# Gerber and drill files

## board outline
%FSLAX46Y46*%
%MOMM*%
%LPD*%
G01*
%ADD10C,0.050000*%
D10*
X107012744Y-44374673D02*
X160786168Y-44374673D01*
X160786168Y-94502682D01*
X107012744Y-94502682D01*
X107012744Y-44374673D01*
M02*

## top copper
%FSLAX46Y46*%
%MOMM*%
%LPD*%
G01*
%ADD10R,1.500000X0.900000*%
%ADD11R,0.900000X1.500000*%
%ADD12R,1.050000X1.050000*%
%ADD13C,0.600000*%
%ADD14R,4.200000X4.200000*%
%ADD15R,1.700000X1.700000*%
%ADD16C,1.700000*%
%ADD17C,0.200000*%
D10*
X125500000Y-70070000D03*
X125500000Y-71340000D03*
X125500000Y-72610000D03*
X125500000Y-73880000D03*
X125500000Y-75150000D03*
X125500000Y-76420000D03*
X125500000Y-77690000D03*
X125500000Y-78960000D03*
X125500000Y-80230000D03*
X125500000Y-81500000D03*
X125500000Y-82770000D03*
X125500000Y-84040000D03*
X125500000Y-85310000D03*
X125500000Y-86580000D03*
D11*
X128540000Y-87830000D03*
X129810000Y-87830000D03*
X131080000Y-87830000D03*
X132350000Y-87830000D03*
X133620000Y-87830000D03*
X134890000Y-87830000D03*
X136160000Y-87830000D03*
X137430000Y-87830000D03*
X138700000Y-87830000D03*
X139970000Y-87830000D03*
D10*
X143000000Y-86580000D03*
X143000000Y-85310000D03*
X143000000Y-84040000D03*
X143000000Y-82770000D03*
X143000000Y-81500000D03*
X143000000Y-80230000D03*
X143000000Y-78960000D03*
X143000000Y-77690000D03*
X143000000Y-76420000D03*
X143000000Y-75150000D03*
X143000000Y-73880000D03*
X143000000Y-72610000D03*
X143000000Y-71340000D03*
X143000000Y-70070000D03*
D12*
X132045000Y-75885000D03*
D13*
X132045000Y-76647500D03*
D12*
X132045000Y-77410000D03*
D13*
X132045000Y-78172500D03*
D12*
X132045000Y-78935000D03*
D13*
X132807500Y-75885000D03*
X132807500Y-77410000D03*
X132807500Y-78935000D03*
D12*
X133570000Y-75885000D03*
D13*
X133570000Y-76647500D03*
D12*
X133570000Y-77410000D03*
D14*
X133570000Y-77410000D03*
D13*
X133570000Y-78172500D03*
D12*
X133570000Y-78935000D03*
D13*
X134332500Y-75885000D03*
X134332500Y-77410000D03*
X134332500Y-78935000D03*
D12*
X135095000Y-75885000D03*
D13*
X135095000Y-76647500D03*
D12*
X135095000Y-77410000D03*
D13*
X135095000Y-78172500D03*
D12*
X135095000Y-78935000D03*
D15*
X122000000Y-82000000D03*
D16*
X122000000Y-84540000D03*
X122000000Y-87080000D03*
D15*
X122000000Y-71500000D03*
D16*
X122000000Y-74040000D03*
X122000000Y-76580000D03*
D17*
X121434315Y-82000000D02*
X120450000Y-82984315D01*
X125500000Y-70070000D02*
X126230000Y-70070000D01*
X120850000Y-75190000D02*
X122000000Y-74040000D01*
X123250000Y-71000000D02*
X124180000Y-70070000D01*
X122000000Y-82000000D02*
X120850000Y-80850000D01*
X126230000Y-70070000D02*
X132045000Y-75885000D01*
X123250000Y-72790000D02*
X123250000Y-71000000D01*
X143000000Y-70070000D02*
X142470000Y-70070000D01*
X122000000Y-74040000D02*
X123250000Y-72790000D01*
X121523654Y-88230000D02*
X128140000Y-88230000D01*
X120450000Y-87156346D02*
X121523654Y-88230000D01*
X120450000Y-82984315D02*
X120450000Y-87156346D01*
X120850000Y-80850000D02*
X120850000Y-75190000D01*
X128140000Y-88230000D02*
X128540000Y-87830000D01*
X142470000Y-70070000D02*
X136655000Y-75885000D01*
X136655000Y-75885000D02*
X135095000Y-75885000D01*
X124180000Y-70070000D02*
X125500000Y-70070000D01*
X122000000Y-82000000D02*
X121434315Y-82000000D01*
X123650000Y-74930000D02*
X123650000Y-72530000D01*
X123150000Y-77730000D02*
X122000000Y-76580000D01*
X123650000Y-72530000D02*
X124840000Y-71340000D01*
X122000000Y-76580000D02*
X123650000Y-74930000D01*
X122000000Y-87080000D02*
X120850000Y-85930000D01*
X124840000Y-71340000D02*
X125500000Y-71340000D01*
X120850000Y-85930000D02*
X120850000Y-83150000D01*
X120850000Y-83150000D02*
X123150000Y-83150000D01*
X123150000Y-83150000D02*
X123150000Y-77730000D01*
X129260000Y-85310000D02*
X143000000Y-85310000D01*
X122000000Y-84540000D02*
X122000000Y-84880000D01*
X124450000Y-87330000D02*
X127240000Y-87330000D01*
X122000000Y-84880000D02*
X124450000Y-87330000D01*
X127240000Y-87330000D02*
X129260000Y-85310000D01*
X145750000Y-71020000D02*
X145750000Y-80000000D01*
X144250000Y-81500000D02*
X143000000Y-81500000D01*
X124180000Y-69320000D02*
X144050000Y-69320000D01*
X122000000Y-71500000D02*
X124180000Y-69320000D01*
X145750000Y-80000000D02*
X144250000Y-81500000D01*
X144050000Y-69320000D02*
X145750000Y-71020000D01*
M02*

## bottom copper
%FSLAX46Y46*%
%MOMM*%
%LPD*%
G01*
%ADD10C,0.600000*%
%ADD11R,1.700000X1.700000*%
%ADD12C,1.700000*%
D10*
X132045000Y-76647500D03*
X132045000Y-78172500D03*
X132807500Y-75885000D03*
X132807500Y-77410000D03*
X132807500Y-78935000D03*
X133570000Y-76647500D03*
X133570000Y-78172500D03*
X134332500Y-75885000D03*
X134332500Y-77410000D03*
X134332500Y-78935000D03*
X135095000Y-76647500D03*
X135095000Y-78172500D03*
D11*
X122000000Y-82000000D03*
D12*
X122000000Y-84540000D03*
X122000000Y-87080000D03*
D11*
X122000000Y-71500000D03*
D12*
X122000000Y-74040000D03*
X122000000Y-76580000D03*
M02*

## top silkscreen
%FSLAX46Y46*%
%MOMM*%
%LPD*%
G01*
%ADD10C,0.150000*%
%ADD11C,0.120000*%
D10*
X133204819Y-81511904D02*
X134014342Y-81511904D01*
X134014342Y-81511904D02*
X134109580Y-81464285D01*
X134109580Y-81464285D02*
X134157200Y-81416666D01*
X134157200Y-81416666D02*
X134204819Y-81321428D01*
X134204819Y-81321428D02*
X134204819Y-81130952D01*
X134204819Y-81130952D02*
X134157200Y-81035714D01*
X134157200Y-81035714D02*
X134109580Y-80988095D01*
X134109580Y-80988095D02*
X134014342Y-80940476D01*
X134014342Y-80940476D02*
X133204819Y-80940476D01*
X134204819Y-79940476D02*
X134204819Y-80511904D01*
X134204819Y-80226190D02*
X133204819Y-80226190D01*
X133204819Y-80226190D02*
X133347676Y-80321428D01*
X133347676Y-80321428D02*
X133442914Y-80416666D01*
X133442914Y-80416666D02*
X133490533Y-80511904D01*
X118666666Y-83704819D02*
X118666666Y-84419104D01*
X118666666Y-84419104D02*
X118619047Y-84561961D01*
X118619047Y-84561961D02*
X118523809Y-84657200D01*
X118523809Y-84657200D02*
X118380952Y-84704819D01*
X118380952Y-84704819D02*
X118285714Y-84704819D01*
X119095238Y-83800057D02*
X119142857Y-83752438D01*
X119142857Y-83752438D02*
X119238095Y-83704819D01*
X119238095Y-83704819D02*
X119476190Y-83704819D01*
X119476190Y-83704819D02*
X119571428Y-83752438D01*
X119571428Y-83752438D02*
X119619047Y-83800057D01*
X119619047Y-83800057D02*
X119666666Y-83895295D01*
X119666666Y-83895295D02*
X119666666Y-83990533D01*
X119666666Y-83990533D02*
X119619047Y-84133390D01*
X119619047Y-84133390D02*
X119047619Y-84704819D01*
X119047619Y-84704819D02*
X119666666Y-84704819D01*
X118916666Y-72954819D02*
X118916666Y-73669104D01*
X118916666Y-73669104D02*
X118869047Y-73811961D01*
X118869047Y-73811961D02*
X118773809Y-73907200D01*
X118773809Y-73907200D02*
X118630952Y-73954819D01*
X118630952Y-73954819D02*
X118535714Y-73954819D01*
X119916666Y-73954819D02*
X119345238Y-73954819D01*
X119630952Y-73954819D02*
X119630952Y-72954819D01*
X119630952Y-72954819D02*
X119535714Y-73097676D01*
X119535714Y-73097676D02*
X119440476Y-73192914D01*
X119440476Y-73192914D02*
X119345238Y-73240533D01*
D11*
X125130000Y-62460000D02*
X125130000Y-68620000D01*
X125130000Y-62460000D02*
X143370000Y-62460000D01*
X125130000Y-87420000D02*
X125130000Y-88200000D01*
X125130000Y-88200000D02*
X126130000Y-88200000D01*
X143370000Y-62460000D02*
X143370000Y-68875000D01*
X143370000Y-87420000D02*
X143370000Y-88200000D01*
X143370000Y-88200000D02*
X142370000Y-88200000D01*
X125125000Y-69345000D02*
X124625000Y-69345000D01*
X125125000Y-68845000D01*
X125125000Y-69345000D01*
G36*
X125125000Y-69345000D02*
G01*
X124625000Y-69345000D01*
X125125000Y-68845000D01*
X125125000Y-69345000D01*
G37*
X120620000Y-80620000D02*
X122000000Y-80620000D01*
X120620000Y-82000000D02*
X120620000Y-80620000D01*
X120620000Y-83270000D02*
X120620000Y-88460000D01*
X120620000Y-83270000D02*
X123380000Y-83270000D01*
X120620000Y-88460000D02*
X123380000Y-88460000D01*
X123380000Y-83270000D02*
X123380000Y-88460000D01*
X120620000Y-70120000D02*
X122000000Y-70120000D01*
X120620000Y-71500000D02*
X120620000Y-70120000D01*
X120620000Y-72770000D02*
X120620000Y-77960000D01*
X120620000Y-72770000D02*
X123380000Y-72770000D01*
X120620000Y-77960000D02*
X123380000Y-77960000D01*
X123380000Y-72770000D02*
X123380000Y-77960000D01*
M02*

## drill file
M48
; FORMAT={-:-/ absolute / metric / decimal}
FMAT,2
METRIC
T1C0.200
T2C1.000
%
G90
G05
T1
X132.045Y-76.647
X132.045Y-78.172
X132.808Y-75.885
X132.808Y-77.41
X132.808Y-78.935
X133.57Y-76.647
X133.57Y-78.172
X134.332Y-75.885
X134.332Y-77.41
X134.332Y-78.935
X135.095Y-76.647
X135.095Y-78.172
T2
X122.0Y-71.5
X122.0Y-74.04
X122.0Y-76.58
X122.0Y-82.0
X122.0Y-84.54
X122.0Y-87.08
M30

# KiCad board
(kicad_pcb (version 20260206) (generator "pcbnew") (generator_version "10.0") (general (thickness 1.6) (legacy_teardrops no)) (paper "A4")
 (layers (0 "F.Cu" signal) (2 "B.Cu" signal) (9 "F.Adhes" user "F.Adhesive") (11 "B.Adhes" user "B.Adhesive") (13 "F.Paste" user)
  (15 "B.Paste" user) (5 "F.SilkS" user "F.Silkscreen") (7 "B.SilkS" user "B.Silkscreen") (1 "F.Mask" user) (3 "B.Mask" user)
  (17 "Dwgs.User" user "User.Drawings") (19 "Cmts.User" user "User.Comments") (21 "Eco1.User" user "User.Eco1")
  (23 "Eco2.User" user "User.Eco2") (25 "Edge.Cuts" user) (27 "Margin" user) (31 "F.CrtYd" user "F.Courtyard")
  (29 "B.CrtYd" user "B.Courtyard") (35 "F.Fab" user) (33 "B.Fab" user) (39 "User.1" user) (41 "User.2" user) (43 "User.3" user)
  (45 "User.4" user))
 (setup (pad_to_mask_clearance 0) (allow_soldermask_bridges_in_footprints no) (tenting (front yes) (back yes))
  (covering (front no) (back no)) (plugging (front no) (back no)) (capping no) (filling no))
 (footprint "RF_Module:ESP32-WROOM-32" (layer "F.Cu") (at 134.25 78.32)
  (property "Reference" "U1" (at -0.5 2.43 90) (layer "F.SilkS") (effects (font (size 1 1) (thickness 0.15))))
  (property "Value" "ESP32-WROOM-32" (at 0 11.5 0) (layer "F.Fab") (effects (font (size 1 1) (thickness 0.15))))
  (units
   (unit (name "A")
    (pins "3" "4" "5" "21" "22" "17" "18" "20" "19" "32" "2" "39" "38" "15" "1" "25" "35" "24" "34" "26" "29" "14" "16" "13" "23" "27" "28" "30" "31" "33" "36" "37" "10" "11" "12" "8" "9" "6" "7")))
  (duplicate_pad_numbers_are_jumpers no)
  (fp_line (start -9.12 -15.86) (end -9.12 -9.7) (stroke (width 0.12) (type solid)) (layer "F.SilkS"))
  (fp_line (start -9.12 -15.86) (end 9.12 -15.86) (stroke (width 0.12) (type solid)) (layer "F.SilkS"))
  (fp_line (start -9.12 9.1) (end -9.12 9.88) (stroke (width 0.12) (type solid)) (layer "F.SilkS"))
  (fp_line (start -9.12 9.88) (end -8.12 9.88) (stroke (width 0.12) (type solid)) (layer "F.SilkS"))
  (fp_line (start 9.12 -15.86) (end 9.12 -9.445) (stroke (width 0.12) (type solid)) (layer "F.SilkS"))
  (fp_line (start 9.12 9.1) (end 9.12 9.88) (stroke (width 0.12) (type solid)) (layer "F.SilkS"))
  (fp_line (start 9.12 9.88) (end 8.12 9.88) (stroke (width 0.12) (type solid)) (layer "F.SilkS"))
  (fp_poly
   (pts (xy -9.125 -8.975) (xy -9.625 -8.975) (xy -9.125 -9.475) (xy -9.125 -8.975)) (stroke (width 0.12) (type solid)) (fill yes)
   (layer "F.SilkS"))
  (pad "1" smd rect (at -8.75 -8.25) (size 1.5 0.9) (layers "F.Cu" "F.Mask" "F.Paste") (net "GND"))
  (pad "2" smd rect (at -8.75 -6.98) (size 1.5 0.9) (layers "F.Cu" "F.Mask" "F.Paste") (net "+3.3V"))
  (pad "3" smd rect (at -8.75 -5.71) (size 1.5 0.9) (layers "F.Cu" "F.Mask" "F.Paste") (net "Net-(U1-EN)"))
  (pad "4" smd rect (at -8.75 -4.44) (size 1.5 0.9) (layers "F.Cu" "F.Mask" "F.Paste") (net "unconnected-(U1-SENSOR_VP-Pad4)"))
  (pad "5" smd rect (at -8.75 -3.17) (size 1.5 0.9) (layers "F.Cu" "F.Mask" "F.Paste") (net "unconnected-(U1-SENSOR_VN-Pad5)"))
  (pad "6" smd rect (at -8.75 -1.9) (size 1.5 0.9) (layers "F.Cu" "F.Mask" "F.Paste") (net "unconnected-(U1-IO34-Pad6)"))
  (pad "7" smd rect (at -8.75 -0.63) (size 1.5 0.9) (layers "F.Cu" "F.Mask" "F.Paste") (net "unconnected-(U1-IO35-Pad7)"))
  (pad "8" smd rect (at -8.75 0.64) (size 1.5 0.9) (layers "F.Cu" "F.Mask" "F.Paste") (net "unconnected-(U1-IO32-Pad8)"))
  (pad "9" smd rect (at -8.75 1.91) (size 1.5 0.9) (layers "F.Cu" "F.Mask" "F.Paste") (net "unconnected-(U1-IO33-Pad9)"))
  (pad "10" smd rect (at -8.75 3.18) (size 1.5 0.9) (layers "F.Cu" "F.Mask" "F.Paste") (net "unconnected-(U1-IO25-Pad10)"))
  (pad "11" smd rect (at -8.75 4.45) (size 1.5 0.9) (layers "F.Cu" "F.Mask" "F.Paste") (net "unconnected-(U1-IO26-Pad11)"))
  (pad "12" smd rect (at -8.75 5.72) (size 1.5 0.9) (layers "F.Cu" "F.Mask" "F.Paste") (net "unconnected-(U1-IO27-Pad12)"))
  (pad "13" smd rect (at -8.75 6.99) (size 1.5 0.9) (layers "F.Cu" "F.Mask" "F.Paste") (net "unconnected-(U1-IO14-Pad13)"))
  (pad "14" smd rect (at -8.75 8.26) (size 1.5 0.9) (layers "F.Cu" "F.Mask" "F.Paste") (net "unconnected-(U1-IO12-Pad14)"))
  (pad "15" smd rect (at -5.71 9.51 90) (size 1.5 0.9) (layers "F.Cu" "F.Mask" "F.Paste") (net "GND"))
  (pad "16" smd rect (at -4.44 9.51 90) (size 1.5 0.9) (layers "F.Cu" "F.Mask" "F.Paste") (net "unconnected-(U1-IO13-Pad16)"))
  (pad "17" smd rect (at -3.17 9.51 90) (size 1.5 0.9) (layers "F.Cu" "F.Mask" "F.Paste") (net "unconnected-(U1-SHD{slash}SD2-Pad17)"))
  (pad "18" smd rect (at -1.9 9.51 90) (size 1.5 0.9) (layers "F.Cu" "F.Mask" "F.Paste") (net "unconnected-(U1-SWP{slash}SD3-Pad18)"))
  (pad "19" smd rect (at -0.63 9.51 90) (size 1.5 0.9) (layers "F.Cu" "F.Mask" "F.Paste") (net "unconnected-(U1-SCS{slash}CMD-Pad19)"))
  (pad "20" smd rect (at 0.64 9.51 90) (size 1.5 0.9) (layers "F.Cu" "F.Mask" "F.Paste") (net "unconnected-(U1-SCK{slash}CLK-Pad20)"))
  (pad "21" smd rect (at 1.91 9.51 90) (size 1.5 0.9) (layers "F.Cu" "F.Mask" "F.Paste") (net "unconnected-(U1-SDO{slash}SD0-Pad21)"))
  (pad "22" smd rect (at 3.18 9.51 90) (size 1.5 0.9) (layers "F.Cu" "F.Mask" "F.Paste") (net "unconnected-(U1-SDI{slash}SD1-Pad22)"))
  (pad "23" smd rect (at 4.45 9.51 90) (size 1.5 0.9) (layers "F.Cu" "F.Mask" "F.Paste") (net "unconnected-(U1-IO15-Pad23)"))
  (pad "24" smd rect (at 5.72 9.51 90) (size 1.5 0.9) (layers "F.Cu" "F.Mask" "F.Paste") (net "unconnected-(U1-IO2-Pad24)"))
  (pad "25" smd rect (at 8.75 8.26) (size 1.5 0.9) (layers "F.Cu" "F.Mask" "F.Paste") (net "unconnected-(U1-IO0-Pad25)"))
  (pad "26" smd rect (at 8.75 6.99) (size 1.5 0.9) (layers "F.Cu" "F.Mask" "F.Paste") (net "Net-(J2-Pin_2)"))
  (pad "27" smd rect (at 8.75 5.72) (size 1.5 0.9) (layers "F.Cu" "F.Mask" "F.Paste") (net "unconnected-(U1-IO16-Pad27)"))
  (pad "28" smd rect (at 8.75 4.45) (size 1.5 0.9) (layers "F.Cu" "F.Mask" "F.Paste") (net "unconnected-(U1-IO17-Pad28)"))
  (pad "29" smd rect (at 8.75 3.18) (size 1.5 0.9) (layers "F.Cu" "F.Mask" "F.Paste") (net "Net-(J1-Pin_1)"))
  (pad "30" smd rect (at 8.75 1.91) (size 1.5 0.9) (layers "F.Cu" "F.Mask" "F.Paste") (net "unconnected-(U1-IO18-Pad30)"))
  (pad "31" smd rect (at 8.75 0.64) (size 1.5 0.9) (layers "F.Cu" "F.Mask" "F.Paste") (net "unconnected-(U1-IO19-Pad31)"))
  (pad "32" smd rect (at 8.75 -0.63) (size 1.5 0.9) (layers "F.Cu" "F.Mask" "F.Paste") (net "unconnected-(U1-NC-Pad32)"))
  (pad "33" smd rect (at 8.75 -1.9) (size 1.5 0.9) (layers "F.Cu" "F.Mask" "F.Paste") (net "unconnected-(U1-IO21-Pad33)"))
  (pad "34" smd rect (at 8.75 -3.17) (size 1.5 0.9) (layers "F.Cu" "F.Mask" "F.Paste") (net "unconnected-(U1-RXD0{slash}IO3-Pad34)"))
  (pad "35" smd rect (at 8.75 -4.44) (size 1.5 0.9) (layers "F.Cu" "F.Mask" "F.Paste") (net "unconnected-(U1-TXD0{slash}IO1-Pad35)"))
  (pad "36" smd rect (at 8.75 -5.71) (size 1.5 0.9) (layers "F.Cu" "F.Mask" "F.Paste") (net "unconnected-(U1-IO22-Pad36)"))
  (pad "37" smd rect (at 8.75 -6.98) (size 1.5 0.9) (layers "F.Cu" "F.Mask" "F.Paste") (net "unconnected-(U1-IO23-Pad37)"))
  (pad "38" smd rect (at 8.75 -8.25) (size 1.5 0.9) (layers "F.Cu" "F.Mask" "F.Paste") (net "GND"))
  (pad "39" smd rect (at -2.205 -2.435) (size 1.05 1.05) (layers "F.Cu" "F.Paste") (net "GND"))
  (pad "39" thru_hole circle (at -2.205 -1.6725) (size 0.6 0.6) (drill 0.2) (layers "*.Cu" "F.Mask") (remove_unused_layers no) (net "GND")
   (zone_connect 2))
  (pad "39" smd rect (at -2.205 -0.91) (size 1.05 1.05) (layers "F.Cu" "F.Paste") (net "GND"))
  (pad "39" thru_hole circle (at -2.205 -0.1475) (size 0.6 0.6) (drill 0.2) (layers "*.Cu" "F.Mask") (remove_unused_layers no) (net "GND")
   (zone_connect 2))
  (pad "39" smd rect (at -2.205 0.615) (size 1.05 1.05) (layers "F.Cu" "F.Paste") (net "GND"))
  (pad "39" thru_hole circle (at -1.4425 -2.435) (size 0.6 0.6) (drill 0.2) (layers "*.Cu" "F.Mask") (remove_unused_layers no) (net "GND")
   (zone_connect 2))
  (pad "39" thru_hole circle (at -1.4425 -0.91) (size 0.6 0.6) (drill 0.2) (layers "*.Cu" "F.Mask") (remove_unused_layers no) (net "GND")
   (zone_connect 2))
  (pad "39" thru_hole circle (at -1.4425 0.615) (size 0.6 0.6) (drill 0.2) (layers "*.Cu" "F.Mask") (remove_unused_layers no) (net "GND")
   (zone_connect 2))
  (pad "39" smd rect (at -0.68 -2.435) (size 1.05 1.05) (layers "F.Cu" "F.Paste") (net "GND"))
  (pad "39" thru_hole circle (at -0.68 -1.6725) (size 0.6 0.6) (drill 0.2) (layers "*.Cu" "F.Mask") (remove_unused_layers no) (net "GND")
   (zone_connect 2))
  (pad "39" smd rect (at -0.68 -0.91) (size 1.05 1.05) (layers "F.Cu" "F.Paste") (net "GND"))
  (pad "39" smd rect (at -0.68 -0.91) (size 4.2 4.2) (layers "F.Cu" "F.Mask") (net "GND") (zone_connect 2))
  (pad "39" thru_hole circle (at -0.68 -0.1475) (size 0.6 0.6) (drill 0.2) (layers "*.Cu" "F.Mask") (remove_unused_layers no) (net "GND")
   (zone_connect 2))
  (pad "39" smd rect (at -0.68 0.615) (size 1.05 1.05) (layers "F.Cu" "F.Paste") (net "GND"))
  (pad "39" thru_hole circle (at 0.0825 -2.435) (size 0.6 0.6) (drill 0.2) (layers "*.Cu" "F.Mask") (remove_unused_layers no) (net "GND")
   (zone_connect 2))
  (pad "39" thru_hole circle (at 0.0825 -0.91) (size 0.6 0.6) (drill 0.2) (layers "*.Cu" "F.Mask") (remove_unused_layers no) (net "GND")
   (zone_connect 2))
  (pad "39" thru_hole circle (at 0.0825 0.615) (size 0.6 0.6) (drill 0.2) (layers "*.Cu" "F.Mask") (remove_unused_layers no) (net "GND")
   (zone_connect 2))
  (pad "39" smd rect (at 0.845 -2.435) (size 1.05 1.05) (layers "F.Cu" "F.Paste") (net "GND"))
  (pad "39" thru_hole circle (at 0.845 -1.6725) (size 0.6 0.6) (drill 0.2) (layers "*.Cu" "F.Mask") (remove_unused_layers no) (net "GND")
   (zone_connect 2))
  (pad "39" smd rect (at 0.845 -0.91) (size 1.05 1.05) (layers "F.Cu" "F.Paste") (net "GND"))
  (pad "39" thru_hole circle (at 0.845 -0.1475) (size 0.6 0.6) (drill 0.2) (layers "*.Cu" "F.Mask") (remove_unused_layers no) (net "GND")
   (zone_connect 2))
  (pad "39" smd rect (at 0.845 0.615) (size 1.05 1.05) (layers "F.Cu" "F.Paste") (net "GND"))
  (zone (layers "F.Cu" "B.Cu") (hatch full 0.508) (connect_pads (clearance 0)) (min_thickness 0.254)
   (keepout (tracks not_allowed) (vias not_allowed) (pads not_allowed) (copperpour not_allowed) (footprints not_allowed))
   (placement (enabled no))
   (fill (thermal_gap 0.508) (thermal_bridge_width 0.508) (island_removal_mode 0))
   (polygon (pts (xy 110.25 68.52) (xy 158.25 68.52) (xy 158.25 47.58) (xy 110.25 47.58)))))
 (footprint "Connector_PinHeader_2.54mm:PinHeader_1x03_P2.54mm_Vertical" (layer "F.Cu") (at 122 82)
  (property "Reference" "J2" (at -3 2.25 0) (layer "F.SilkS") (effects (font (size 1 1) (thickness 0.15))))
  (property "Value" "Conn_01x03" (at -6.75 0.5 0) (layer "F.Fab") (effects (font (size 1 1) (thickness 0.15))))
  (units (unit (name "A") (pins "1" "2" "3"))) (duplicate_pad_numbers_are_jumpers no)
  (fp_line (start -1.38 -1.38) (end 0 -1.38) (stroke (width 0.12) (type solid)) (layer "F.SilkS"))
  (fp_line (start -1.38 0) (end -1.38 -1.38) (stroke (width 0.12) (type solid)) (layer "F.SilkS"))
  (fp_line (start -1.38 1.27) (end -1.38 6.46) (stroke (width 0.12) (type solid)) (layer "F.SilkS"))
  (fp_line (start -1.38 1.27) (end 1.38 1.27) (stroke (width 0.12) (type solid)) (layer "F.SilkS"))
  (fp_line (start -1.38 6.46) (end 1.38 6.46) (stroke (width 0.12) (type solid)) (layer "F.SilkS"))
  (fp_line (start 1.38 1.27) (end 1.38 6.46) (stroke (width 0.12) (type solid)) (layer "F.SilkS"))
  (pad "1" thru_hole rect (at 0 0) (size 1.7 1.7) (drill 1) (layers "*.Cu" "*.Mask") (remove_unused_layers no) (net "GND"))
  (pad "2" thru_hole circle (at 0 2.54) (size 1.7 1.7) (drill 1) (layers "*.Cu" "*.Mask") (remove_unused_layers no) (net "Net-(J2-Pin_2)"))
  (pad "3" thru_hole circle (at 0 5.08) (size 1.7 1.7) (drill 1) (layers "*.Cu" "*.Mask") (remove_unused_layers no) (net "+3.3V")))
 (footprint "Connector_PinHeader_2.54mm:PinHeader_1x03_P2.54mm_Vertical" (layer "F.Cu") (at 122 71.5)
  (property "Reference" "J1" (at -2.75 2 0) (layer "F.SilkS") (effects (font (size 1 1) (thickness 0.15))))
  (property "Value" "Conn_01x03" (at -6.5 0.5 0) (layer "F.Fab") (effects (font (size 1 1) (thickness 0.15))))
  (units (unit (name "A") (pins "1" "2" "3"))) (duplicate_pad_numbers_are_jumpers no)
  (fp_line (start -1.38 -1.38) (end 0 -1.38) (stroke (width 0.12) (type solid)) (layer "F.SilkS"))
  (fp_line (start -1.38 0) (end -1.38 -1.38) (stroke (width 0.12) (type solid)) (layer "F.SilkS"))
  (fp_line (start -1.38 1.27) (end -1.38 6.46) (stroke (width 0.12) (type solid)) (layer "F.SilkS"))
  (fp_line (start -1.38 1.27) (end 1.38 1.27) (stroke (width 0.12) (type solid)) (layer "F.SilkS"))
  (fp_line (start -1.38 6.46) (end 1.38 6.46) (stroke (width 0.12) (type solid)) (layer "F.SilkS"))
  (fp_line (start 1.38 1.27) (end 1.38 6.46) (stroke (width 0.12) (type solid)) (layer "F.SilkS"))
  (pad "1" thru_hole rect (at 0 0) (size 1.7 1.7) (drill 1) (layers "*.Cu" "*.Mask") (remove_unused_layers no) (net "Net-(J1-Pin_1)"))
  (pad "2" thru_hole circle (at 0 2.54) (size 1.7 1.7) (drill 1) (layers "*.Cu" "*.Mask") (remove_unused_layers no) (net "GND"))
  (pad "3" thru_hole circle (at 0 5.08) (size 1.7 1.7) (drill 1) (layers "*.Cu" "*.Mask") (remove_unused_layers no) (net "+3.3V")))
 (gr_rect (start 107.012744 44.374673) (end 160.786168 94.502682) (stroke (width 0.05) (type default)) (fill no) (layer "Edge.Cuts"))
 (segment (start 121.434315 82) (end 120.45 82.984315) (width 0.2) (layer "F.Cu") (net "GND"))
 (segment (start 125.5 70.07) (end 126.23 70.07) (width 0.2) (layer "F.Cu") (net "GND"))
 (segment (start 120.85 75.19) (end 122 74.04) (width 0.2) (layer "F.Cu") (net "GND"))
 (segment (start 123.25 71) (end 124.18 70.07) (width 0.2) (layer "F.Cu") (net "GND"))
 (segment (start 122 82) (end 120.85 80.85) (width 0.2) (layer "F.Cu") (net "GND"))
 (segment (start 126.23 70.07) (end 132.045 75.885) (width 0.2) (layer "F.Cu") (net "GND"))
 (segment (start 123.25 72.79) (end 123.25 71) (width 0.2) (layer "F.Cu") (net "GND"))
 (segment (start 143 70.07) (end 142.47 70.07) (width 0.2) (layer "F.Cu") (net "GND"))
 (segment (start 122 74.04) (end 123.25 72.79) (width 0.2) (layer "F.Cu") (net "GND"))
 (segment (start 121.523654 88.23) (end 128.14 88.23) (width 0.2) (layer "F.Cu") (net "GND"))
 (segment (start 120.45 87.156346) (end 121.523654 88.23) (width 0.2) (layer "F.Cu") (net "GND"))
 (segment (start 120.45 82.984315) (end 120.45 87.156346) (width 0.2) (layer "F.Cu") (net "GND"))
 (segment (start 120.85 80.85) (end 120.85 75.19) (width 0.2) (layer "F.Cu") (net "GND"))
 (segment (start 128.14 88.23) (end 128.54 87.83) (width 0.2) (layer "F.Cu") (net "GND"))
 (segment (start 142.47 70.07) (end 136.655 75.885) (width 0.2) (layer "F.Cu") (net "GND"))
 (segment (start 136.655 75.885) (end 135.095 75.885) (width 0.2) (layer "F.Cu") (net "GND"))
 (segment (start 124.18 70.07) (end 125.5 70.07) (width 0.2) (layer "F.Cu") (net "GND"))
 (segment (start 122 82) (end 121.434315 82) (width 0.2) (layer "F.Cu") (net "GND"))
 (segment (start 123.65 74.93) (end 123.65 72.53) (width 0.2) (layer "F.Cu") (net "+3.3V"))
 (segment (start 123.15 77.73) (end 122 76.58) (width 0.2) (layer "F.Cu") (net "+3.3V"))
 (segment (start 123.65 72.53) (end 124.84 71.34) (width 0.2) (layer "F.Cu") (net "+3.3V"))
 (segment (start 122 76.58) (end 123.65 74.93) (width 0.2) (layer "F.Cu") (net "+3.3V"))
 (segment (start 122 87.08) (end 120.85 85.93) (width 0.2) (layer "F.Cu") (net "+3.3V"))
 (segment (start 124.84 71.34) (end 125.5 71.34) (width 0.2) (layer "F.Cu") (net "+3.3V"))
 (segment (start 120.85 85.93) (end 120.85 83.15) (width 0.2) (layer "F.Cu") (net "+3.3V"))
 (segment (start 120.85 83.15) (end 123.15 83.15) (width 0.2) (layer "F.Cu") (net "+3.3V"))
 (segment (start 123.15 83.15) (end 123.15 77.73) (width 0.2) (layer "F.Cu") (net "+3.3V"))
 (segment (start 129.26 85.31) (end 143 85.31) (width 0.2) (layer "F.Cu") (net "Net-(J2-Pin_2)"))
 (segment (start 122 84.54) (end 122 84.88) (width 0.2) (layer "F.Cu") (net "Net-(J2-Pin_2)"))
 (segment (start 124.45 87.33) (end 127.24 87.33) (width 0.2) (layer "F.Cu") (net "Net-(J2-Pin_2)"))
 (segment (start 122 84.88) (end 124.45 87.33) (width 0.2) (layer "F.Cu") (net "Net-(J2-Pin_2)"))
 (segment (start 127.24 87.33) (end 129.26 85.31) (width 0.2) (layer "F.Cu") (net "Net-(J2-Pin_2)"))
 (segment (start 145.75 71.02) (end 145.75 80) (width 0.2) (layer "F.Cu") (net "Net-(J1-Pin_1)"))
 (segment (start 144.25 81.5) (end 143 81.5) (width 0.2) (layer "F.Cu") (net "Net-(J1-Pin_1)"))
 (segment (start 124.18 69.32) (end 144.05 69.32) (width 0.2) (layer "F.Cu") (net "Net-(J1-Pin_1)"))
 (segment (start 122 71.5) (end 124.18 69.32) (width 0.2) (layer "F.Cu") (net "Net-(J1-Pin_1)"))
 (segment (start 145.75 80) (end 144.25 81.5) (width 0.2) (layer "F.Cu") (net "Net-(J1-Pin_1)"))
 (segment (start 144.05 69.32) (end 145.75 71.02) (width 0.2) (layer "F.Cu") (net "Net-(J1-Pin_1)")))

